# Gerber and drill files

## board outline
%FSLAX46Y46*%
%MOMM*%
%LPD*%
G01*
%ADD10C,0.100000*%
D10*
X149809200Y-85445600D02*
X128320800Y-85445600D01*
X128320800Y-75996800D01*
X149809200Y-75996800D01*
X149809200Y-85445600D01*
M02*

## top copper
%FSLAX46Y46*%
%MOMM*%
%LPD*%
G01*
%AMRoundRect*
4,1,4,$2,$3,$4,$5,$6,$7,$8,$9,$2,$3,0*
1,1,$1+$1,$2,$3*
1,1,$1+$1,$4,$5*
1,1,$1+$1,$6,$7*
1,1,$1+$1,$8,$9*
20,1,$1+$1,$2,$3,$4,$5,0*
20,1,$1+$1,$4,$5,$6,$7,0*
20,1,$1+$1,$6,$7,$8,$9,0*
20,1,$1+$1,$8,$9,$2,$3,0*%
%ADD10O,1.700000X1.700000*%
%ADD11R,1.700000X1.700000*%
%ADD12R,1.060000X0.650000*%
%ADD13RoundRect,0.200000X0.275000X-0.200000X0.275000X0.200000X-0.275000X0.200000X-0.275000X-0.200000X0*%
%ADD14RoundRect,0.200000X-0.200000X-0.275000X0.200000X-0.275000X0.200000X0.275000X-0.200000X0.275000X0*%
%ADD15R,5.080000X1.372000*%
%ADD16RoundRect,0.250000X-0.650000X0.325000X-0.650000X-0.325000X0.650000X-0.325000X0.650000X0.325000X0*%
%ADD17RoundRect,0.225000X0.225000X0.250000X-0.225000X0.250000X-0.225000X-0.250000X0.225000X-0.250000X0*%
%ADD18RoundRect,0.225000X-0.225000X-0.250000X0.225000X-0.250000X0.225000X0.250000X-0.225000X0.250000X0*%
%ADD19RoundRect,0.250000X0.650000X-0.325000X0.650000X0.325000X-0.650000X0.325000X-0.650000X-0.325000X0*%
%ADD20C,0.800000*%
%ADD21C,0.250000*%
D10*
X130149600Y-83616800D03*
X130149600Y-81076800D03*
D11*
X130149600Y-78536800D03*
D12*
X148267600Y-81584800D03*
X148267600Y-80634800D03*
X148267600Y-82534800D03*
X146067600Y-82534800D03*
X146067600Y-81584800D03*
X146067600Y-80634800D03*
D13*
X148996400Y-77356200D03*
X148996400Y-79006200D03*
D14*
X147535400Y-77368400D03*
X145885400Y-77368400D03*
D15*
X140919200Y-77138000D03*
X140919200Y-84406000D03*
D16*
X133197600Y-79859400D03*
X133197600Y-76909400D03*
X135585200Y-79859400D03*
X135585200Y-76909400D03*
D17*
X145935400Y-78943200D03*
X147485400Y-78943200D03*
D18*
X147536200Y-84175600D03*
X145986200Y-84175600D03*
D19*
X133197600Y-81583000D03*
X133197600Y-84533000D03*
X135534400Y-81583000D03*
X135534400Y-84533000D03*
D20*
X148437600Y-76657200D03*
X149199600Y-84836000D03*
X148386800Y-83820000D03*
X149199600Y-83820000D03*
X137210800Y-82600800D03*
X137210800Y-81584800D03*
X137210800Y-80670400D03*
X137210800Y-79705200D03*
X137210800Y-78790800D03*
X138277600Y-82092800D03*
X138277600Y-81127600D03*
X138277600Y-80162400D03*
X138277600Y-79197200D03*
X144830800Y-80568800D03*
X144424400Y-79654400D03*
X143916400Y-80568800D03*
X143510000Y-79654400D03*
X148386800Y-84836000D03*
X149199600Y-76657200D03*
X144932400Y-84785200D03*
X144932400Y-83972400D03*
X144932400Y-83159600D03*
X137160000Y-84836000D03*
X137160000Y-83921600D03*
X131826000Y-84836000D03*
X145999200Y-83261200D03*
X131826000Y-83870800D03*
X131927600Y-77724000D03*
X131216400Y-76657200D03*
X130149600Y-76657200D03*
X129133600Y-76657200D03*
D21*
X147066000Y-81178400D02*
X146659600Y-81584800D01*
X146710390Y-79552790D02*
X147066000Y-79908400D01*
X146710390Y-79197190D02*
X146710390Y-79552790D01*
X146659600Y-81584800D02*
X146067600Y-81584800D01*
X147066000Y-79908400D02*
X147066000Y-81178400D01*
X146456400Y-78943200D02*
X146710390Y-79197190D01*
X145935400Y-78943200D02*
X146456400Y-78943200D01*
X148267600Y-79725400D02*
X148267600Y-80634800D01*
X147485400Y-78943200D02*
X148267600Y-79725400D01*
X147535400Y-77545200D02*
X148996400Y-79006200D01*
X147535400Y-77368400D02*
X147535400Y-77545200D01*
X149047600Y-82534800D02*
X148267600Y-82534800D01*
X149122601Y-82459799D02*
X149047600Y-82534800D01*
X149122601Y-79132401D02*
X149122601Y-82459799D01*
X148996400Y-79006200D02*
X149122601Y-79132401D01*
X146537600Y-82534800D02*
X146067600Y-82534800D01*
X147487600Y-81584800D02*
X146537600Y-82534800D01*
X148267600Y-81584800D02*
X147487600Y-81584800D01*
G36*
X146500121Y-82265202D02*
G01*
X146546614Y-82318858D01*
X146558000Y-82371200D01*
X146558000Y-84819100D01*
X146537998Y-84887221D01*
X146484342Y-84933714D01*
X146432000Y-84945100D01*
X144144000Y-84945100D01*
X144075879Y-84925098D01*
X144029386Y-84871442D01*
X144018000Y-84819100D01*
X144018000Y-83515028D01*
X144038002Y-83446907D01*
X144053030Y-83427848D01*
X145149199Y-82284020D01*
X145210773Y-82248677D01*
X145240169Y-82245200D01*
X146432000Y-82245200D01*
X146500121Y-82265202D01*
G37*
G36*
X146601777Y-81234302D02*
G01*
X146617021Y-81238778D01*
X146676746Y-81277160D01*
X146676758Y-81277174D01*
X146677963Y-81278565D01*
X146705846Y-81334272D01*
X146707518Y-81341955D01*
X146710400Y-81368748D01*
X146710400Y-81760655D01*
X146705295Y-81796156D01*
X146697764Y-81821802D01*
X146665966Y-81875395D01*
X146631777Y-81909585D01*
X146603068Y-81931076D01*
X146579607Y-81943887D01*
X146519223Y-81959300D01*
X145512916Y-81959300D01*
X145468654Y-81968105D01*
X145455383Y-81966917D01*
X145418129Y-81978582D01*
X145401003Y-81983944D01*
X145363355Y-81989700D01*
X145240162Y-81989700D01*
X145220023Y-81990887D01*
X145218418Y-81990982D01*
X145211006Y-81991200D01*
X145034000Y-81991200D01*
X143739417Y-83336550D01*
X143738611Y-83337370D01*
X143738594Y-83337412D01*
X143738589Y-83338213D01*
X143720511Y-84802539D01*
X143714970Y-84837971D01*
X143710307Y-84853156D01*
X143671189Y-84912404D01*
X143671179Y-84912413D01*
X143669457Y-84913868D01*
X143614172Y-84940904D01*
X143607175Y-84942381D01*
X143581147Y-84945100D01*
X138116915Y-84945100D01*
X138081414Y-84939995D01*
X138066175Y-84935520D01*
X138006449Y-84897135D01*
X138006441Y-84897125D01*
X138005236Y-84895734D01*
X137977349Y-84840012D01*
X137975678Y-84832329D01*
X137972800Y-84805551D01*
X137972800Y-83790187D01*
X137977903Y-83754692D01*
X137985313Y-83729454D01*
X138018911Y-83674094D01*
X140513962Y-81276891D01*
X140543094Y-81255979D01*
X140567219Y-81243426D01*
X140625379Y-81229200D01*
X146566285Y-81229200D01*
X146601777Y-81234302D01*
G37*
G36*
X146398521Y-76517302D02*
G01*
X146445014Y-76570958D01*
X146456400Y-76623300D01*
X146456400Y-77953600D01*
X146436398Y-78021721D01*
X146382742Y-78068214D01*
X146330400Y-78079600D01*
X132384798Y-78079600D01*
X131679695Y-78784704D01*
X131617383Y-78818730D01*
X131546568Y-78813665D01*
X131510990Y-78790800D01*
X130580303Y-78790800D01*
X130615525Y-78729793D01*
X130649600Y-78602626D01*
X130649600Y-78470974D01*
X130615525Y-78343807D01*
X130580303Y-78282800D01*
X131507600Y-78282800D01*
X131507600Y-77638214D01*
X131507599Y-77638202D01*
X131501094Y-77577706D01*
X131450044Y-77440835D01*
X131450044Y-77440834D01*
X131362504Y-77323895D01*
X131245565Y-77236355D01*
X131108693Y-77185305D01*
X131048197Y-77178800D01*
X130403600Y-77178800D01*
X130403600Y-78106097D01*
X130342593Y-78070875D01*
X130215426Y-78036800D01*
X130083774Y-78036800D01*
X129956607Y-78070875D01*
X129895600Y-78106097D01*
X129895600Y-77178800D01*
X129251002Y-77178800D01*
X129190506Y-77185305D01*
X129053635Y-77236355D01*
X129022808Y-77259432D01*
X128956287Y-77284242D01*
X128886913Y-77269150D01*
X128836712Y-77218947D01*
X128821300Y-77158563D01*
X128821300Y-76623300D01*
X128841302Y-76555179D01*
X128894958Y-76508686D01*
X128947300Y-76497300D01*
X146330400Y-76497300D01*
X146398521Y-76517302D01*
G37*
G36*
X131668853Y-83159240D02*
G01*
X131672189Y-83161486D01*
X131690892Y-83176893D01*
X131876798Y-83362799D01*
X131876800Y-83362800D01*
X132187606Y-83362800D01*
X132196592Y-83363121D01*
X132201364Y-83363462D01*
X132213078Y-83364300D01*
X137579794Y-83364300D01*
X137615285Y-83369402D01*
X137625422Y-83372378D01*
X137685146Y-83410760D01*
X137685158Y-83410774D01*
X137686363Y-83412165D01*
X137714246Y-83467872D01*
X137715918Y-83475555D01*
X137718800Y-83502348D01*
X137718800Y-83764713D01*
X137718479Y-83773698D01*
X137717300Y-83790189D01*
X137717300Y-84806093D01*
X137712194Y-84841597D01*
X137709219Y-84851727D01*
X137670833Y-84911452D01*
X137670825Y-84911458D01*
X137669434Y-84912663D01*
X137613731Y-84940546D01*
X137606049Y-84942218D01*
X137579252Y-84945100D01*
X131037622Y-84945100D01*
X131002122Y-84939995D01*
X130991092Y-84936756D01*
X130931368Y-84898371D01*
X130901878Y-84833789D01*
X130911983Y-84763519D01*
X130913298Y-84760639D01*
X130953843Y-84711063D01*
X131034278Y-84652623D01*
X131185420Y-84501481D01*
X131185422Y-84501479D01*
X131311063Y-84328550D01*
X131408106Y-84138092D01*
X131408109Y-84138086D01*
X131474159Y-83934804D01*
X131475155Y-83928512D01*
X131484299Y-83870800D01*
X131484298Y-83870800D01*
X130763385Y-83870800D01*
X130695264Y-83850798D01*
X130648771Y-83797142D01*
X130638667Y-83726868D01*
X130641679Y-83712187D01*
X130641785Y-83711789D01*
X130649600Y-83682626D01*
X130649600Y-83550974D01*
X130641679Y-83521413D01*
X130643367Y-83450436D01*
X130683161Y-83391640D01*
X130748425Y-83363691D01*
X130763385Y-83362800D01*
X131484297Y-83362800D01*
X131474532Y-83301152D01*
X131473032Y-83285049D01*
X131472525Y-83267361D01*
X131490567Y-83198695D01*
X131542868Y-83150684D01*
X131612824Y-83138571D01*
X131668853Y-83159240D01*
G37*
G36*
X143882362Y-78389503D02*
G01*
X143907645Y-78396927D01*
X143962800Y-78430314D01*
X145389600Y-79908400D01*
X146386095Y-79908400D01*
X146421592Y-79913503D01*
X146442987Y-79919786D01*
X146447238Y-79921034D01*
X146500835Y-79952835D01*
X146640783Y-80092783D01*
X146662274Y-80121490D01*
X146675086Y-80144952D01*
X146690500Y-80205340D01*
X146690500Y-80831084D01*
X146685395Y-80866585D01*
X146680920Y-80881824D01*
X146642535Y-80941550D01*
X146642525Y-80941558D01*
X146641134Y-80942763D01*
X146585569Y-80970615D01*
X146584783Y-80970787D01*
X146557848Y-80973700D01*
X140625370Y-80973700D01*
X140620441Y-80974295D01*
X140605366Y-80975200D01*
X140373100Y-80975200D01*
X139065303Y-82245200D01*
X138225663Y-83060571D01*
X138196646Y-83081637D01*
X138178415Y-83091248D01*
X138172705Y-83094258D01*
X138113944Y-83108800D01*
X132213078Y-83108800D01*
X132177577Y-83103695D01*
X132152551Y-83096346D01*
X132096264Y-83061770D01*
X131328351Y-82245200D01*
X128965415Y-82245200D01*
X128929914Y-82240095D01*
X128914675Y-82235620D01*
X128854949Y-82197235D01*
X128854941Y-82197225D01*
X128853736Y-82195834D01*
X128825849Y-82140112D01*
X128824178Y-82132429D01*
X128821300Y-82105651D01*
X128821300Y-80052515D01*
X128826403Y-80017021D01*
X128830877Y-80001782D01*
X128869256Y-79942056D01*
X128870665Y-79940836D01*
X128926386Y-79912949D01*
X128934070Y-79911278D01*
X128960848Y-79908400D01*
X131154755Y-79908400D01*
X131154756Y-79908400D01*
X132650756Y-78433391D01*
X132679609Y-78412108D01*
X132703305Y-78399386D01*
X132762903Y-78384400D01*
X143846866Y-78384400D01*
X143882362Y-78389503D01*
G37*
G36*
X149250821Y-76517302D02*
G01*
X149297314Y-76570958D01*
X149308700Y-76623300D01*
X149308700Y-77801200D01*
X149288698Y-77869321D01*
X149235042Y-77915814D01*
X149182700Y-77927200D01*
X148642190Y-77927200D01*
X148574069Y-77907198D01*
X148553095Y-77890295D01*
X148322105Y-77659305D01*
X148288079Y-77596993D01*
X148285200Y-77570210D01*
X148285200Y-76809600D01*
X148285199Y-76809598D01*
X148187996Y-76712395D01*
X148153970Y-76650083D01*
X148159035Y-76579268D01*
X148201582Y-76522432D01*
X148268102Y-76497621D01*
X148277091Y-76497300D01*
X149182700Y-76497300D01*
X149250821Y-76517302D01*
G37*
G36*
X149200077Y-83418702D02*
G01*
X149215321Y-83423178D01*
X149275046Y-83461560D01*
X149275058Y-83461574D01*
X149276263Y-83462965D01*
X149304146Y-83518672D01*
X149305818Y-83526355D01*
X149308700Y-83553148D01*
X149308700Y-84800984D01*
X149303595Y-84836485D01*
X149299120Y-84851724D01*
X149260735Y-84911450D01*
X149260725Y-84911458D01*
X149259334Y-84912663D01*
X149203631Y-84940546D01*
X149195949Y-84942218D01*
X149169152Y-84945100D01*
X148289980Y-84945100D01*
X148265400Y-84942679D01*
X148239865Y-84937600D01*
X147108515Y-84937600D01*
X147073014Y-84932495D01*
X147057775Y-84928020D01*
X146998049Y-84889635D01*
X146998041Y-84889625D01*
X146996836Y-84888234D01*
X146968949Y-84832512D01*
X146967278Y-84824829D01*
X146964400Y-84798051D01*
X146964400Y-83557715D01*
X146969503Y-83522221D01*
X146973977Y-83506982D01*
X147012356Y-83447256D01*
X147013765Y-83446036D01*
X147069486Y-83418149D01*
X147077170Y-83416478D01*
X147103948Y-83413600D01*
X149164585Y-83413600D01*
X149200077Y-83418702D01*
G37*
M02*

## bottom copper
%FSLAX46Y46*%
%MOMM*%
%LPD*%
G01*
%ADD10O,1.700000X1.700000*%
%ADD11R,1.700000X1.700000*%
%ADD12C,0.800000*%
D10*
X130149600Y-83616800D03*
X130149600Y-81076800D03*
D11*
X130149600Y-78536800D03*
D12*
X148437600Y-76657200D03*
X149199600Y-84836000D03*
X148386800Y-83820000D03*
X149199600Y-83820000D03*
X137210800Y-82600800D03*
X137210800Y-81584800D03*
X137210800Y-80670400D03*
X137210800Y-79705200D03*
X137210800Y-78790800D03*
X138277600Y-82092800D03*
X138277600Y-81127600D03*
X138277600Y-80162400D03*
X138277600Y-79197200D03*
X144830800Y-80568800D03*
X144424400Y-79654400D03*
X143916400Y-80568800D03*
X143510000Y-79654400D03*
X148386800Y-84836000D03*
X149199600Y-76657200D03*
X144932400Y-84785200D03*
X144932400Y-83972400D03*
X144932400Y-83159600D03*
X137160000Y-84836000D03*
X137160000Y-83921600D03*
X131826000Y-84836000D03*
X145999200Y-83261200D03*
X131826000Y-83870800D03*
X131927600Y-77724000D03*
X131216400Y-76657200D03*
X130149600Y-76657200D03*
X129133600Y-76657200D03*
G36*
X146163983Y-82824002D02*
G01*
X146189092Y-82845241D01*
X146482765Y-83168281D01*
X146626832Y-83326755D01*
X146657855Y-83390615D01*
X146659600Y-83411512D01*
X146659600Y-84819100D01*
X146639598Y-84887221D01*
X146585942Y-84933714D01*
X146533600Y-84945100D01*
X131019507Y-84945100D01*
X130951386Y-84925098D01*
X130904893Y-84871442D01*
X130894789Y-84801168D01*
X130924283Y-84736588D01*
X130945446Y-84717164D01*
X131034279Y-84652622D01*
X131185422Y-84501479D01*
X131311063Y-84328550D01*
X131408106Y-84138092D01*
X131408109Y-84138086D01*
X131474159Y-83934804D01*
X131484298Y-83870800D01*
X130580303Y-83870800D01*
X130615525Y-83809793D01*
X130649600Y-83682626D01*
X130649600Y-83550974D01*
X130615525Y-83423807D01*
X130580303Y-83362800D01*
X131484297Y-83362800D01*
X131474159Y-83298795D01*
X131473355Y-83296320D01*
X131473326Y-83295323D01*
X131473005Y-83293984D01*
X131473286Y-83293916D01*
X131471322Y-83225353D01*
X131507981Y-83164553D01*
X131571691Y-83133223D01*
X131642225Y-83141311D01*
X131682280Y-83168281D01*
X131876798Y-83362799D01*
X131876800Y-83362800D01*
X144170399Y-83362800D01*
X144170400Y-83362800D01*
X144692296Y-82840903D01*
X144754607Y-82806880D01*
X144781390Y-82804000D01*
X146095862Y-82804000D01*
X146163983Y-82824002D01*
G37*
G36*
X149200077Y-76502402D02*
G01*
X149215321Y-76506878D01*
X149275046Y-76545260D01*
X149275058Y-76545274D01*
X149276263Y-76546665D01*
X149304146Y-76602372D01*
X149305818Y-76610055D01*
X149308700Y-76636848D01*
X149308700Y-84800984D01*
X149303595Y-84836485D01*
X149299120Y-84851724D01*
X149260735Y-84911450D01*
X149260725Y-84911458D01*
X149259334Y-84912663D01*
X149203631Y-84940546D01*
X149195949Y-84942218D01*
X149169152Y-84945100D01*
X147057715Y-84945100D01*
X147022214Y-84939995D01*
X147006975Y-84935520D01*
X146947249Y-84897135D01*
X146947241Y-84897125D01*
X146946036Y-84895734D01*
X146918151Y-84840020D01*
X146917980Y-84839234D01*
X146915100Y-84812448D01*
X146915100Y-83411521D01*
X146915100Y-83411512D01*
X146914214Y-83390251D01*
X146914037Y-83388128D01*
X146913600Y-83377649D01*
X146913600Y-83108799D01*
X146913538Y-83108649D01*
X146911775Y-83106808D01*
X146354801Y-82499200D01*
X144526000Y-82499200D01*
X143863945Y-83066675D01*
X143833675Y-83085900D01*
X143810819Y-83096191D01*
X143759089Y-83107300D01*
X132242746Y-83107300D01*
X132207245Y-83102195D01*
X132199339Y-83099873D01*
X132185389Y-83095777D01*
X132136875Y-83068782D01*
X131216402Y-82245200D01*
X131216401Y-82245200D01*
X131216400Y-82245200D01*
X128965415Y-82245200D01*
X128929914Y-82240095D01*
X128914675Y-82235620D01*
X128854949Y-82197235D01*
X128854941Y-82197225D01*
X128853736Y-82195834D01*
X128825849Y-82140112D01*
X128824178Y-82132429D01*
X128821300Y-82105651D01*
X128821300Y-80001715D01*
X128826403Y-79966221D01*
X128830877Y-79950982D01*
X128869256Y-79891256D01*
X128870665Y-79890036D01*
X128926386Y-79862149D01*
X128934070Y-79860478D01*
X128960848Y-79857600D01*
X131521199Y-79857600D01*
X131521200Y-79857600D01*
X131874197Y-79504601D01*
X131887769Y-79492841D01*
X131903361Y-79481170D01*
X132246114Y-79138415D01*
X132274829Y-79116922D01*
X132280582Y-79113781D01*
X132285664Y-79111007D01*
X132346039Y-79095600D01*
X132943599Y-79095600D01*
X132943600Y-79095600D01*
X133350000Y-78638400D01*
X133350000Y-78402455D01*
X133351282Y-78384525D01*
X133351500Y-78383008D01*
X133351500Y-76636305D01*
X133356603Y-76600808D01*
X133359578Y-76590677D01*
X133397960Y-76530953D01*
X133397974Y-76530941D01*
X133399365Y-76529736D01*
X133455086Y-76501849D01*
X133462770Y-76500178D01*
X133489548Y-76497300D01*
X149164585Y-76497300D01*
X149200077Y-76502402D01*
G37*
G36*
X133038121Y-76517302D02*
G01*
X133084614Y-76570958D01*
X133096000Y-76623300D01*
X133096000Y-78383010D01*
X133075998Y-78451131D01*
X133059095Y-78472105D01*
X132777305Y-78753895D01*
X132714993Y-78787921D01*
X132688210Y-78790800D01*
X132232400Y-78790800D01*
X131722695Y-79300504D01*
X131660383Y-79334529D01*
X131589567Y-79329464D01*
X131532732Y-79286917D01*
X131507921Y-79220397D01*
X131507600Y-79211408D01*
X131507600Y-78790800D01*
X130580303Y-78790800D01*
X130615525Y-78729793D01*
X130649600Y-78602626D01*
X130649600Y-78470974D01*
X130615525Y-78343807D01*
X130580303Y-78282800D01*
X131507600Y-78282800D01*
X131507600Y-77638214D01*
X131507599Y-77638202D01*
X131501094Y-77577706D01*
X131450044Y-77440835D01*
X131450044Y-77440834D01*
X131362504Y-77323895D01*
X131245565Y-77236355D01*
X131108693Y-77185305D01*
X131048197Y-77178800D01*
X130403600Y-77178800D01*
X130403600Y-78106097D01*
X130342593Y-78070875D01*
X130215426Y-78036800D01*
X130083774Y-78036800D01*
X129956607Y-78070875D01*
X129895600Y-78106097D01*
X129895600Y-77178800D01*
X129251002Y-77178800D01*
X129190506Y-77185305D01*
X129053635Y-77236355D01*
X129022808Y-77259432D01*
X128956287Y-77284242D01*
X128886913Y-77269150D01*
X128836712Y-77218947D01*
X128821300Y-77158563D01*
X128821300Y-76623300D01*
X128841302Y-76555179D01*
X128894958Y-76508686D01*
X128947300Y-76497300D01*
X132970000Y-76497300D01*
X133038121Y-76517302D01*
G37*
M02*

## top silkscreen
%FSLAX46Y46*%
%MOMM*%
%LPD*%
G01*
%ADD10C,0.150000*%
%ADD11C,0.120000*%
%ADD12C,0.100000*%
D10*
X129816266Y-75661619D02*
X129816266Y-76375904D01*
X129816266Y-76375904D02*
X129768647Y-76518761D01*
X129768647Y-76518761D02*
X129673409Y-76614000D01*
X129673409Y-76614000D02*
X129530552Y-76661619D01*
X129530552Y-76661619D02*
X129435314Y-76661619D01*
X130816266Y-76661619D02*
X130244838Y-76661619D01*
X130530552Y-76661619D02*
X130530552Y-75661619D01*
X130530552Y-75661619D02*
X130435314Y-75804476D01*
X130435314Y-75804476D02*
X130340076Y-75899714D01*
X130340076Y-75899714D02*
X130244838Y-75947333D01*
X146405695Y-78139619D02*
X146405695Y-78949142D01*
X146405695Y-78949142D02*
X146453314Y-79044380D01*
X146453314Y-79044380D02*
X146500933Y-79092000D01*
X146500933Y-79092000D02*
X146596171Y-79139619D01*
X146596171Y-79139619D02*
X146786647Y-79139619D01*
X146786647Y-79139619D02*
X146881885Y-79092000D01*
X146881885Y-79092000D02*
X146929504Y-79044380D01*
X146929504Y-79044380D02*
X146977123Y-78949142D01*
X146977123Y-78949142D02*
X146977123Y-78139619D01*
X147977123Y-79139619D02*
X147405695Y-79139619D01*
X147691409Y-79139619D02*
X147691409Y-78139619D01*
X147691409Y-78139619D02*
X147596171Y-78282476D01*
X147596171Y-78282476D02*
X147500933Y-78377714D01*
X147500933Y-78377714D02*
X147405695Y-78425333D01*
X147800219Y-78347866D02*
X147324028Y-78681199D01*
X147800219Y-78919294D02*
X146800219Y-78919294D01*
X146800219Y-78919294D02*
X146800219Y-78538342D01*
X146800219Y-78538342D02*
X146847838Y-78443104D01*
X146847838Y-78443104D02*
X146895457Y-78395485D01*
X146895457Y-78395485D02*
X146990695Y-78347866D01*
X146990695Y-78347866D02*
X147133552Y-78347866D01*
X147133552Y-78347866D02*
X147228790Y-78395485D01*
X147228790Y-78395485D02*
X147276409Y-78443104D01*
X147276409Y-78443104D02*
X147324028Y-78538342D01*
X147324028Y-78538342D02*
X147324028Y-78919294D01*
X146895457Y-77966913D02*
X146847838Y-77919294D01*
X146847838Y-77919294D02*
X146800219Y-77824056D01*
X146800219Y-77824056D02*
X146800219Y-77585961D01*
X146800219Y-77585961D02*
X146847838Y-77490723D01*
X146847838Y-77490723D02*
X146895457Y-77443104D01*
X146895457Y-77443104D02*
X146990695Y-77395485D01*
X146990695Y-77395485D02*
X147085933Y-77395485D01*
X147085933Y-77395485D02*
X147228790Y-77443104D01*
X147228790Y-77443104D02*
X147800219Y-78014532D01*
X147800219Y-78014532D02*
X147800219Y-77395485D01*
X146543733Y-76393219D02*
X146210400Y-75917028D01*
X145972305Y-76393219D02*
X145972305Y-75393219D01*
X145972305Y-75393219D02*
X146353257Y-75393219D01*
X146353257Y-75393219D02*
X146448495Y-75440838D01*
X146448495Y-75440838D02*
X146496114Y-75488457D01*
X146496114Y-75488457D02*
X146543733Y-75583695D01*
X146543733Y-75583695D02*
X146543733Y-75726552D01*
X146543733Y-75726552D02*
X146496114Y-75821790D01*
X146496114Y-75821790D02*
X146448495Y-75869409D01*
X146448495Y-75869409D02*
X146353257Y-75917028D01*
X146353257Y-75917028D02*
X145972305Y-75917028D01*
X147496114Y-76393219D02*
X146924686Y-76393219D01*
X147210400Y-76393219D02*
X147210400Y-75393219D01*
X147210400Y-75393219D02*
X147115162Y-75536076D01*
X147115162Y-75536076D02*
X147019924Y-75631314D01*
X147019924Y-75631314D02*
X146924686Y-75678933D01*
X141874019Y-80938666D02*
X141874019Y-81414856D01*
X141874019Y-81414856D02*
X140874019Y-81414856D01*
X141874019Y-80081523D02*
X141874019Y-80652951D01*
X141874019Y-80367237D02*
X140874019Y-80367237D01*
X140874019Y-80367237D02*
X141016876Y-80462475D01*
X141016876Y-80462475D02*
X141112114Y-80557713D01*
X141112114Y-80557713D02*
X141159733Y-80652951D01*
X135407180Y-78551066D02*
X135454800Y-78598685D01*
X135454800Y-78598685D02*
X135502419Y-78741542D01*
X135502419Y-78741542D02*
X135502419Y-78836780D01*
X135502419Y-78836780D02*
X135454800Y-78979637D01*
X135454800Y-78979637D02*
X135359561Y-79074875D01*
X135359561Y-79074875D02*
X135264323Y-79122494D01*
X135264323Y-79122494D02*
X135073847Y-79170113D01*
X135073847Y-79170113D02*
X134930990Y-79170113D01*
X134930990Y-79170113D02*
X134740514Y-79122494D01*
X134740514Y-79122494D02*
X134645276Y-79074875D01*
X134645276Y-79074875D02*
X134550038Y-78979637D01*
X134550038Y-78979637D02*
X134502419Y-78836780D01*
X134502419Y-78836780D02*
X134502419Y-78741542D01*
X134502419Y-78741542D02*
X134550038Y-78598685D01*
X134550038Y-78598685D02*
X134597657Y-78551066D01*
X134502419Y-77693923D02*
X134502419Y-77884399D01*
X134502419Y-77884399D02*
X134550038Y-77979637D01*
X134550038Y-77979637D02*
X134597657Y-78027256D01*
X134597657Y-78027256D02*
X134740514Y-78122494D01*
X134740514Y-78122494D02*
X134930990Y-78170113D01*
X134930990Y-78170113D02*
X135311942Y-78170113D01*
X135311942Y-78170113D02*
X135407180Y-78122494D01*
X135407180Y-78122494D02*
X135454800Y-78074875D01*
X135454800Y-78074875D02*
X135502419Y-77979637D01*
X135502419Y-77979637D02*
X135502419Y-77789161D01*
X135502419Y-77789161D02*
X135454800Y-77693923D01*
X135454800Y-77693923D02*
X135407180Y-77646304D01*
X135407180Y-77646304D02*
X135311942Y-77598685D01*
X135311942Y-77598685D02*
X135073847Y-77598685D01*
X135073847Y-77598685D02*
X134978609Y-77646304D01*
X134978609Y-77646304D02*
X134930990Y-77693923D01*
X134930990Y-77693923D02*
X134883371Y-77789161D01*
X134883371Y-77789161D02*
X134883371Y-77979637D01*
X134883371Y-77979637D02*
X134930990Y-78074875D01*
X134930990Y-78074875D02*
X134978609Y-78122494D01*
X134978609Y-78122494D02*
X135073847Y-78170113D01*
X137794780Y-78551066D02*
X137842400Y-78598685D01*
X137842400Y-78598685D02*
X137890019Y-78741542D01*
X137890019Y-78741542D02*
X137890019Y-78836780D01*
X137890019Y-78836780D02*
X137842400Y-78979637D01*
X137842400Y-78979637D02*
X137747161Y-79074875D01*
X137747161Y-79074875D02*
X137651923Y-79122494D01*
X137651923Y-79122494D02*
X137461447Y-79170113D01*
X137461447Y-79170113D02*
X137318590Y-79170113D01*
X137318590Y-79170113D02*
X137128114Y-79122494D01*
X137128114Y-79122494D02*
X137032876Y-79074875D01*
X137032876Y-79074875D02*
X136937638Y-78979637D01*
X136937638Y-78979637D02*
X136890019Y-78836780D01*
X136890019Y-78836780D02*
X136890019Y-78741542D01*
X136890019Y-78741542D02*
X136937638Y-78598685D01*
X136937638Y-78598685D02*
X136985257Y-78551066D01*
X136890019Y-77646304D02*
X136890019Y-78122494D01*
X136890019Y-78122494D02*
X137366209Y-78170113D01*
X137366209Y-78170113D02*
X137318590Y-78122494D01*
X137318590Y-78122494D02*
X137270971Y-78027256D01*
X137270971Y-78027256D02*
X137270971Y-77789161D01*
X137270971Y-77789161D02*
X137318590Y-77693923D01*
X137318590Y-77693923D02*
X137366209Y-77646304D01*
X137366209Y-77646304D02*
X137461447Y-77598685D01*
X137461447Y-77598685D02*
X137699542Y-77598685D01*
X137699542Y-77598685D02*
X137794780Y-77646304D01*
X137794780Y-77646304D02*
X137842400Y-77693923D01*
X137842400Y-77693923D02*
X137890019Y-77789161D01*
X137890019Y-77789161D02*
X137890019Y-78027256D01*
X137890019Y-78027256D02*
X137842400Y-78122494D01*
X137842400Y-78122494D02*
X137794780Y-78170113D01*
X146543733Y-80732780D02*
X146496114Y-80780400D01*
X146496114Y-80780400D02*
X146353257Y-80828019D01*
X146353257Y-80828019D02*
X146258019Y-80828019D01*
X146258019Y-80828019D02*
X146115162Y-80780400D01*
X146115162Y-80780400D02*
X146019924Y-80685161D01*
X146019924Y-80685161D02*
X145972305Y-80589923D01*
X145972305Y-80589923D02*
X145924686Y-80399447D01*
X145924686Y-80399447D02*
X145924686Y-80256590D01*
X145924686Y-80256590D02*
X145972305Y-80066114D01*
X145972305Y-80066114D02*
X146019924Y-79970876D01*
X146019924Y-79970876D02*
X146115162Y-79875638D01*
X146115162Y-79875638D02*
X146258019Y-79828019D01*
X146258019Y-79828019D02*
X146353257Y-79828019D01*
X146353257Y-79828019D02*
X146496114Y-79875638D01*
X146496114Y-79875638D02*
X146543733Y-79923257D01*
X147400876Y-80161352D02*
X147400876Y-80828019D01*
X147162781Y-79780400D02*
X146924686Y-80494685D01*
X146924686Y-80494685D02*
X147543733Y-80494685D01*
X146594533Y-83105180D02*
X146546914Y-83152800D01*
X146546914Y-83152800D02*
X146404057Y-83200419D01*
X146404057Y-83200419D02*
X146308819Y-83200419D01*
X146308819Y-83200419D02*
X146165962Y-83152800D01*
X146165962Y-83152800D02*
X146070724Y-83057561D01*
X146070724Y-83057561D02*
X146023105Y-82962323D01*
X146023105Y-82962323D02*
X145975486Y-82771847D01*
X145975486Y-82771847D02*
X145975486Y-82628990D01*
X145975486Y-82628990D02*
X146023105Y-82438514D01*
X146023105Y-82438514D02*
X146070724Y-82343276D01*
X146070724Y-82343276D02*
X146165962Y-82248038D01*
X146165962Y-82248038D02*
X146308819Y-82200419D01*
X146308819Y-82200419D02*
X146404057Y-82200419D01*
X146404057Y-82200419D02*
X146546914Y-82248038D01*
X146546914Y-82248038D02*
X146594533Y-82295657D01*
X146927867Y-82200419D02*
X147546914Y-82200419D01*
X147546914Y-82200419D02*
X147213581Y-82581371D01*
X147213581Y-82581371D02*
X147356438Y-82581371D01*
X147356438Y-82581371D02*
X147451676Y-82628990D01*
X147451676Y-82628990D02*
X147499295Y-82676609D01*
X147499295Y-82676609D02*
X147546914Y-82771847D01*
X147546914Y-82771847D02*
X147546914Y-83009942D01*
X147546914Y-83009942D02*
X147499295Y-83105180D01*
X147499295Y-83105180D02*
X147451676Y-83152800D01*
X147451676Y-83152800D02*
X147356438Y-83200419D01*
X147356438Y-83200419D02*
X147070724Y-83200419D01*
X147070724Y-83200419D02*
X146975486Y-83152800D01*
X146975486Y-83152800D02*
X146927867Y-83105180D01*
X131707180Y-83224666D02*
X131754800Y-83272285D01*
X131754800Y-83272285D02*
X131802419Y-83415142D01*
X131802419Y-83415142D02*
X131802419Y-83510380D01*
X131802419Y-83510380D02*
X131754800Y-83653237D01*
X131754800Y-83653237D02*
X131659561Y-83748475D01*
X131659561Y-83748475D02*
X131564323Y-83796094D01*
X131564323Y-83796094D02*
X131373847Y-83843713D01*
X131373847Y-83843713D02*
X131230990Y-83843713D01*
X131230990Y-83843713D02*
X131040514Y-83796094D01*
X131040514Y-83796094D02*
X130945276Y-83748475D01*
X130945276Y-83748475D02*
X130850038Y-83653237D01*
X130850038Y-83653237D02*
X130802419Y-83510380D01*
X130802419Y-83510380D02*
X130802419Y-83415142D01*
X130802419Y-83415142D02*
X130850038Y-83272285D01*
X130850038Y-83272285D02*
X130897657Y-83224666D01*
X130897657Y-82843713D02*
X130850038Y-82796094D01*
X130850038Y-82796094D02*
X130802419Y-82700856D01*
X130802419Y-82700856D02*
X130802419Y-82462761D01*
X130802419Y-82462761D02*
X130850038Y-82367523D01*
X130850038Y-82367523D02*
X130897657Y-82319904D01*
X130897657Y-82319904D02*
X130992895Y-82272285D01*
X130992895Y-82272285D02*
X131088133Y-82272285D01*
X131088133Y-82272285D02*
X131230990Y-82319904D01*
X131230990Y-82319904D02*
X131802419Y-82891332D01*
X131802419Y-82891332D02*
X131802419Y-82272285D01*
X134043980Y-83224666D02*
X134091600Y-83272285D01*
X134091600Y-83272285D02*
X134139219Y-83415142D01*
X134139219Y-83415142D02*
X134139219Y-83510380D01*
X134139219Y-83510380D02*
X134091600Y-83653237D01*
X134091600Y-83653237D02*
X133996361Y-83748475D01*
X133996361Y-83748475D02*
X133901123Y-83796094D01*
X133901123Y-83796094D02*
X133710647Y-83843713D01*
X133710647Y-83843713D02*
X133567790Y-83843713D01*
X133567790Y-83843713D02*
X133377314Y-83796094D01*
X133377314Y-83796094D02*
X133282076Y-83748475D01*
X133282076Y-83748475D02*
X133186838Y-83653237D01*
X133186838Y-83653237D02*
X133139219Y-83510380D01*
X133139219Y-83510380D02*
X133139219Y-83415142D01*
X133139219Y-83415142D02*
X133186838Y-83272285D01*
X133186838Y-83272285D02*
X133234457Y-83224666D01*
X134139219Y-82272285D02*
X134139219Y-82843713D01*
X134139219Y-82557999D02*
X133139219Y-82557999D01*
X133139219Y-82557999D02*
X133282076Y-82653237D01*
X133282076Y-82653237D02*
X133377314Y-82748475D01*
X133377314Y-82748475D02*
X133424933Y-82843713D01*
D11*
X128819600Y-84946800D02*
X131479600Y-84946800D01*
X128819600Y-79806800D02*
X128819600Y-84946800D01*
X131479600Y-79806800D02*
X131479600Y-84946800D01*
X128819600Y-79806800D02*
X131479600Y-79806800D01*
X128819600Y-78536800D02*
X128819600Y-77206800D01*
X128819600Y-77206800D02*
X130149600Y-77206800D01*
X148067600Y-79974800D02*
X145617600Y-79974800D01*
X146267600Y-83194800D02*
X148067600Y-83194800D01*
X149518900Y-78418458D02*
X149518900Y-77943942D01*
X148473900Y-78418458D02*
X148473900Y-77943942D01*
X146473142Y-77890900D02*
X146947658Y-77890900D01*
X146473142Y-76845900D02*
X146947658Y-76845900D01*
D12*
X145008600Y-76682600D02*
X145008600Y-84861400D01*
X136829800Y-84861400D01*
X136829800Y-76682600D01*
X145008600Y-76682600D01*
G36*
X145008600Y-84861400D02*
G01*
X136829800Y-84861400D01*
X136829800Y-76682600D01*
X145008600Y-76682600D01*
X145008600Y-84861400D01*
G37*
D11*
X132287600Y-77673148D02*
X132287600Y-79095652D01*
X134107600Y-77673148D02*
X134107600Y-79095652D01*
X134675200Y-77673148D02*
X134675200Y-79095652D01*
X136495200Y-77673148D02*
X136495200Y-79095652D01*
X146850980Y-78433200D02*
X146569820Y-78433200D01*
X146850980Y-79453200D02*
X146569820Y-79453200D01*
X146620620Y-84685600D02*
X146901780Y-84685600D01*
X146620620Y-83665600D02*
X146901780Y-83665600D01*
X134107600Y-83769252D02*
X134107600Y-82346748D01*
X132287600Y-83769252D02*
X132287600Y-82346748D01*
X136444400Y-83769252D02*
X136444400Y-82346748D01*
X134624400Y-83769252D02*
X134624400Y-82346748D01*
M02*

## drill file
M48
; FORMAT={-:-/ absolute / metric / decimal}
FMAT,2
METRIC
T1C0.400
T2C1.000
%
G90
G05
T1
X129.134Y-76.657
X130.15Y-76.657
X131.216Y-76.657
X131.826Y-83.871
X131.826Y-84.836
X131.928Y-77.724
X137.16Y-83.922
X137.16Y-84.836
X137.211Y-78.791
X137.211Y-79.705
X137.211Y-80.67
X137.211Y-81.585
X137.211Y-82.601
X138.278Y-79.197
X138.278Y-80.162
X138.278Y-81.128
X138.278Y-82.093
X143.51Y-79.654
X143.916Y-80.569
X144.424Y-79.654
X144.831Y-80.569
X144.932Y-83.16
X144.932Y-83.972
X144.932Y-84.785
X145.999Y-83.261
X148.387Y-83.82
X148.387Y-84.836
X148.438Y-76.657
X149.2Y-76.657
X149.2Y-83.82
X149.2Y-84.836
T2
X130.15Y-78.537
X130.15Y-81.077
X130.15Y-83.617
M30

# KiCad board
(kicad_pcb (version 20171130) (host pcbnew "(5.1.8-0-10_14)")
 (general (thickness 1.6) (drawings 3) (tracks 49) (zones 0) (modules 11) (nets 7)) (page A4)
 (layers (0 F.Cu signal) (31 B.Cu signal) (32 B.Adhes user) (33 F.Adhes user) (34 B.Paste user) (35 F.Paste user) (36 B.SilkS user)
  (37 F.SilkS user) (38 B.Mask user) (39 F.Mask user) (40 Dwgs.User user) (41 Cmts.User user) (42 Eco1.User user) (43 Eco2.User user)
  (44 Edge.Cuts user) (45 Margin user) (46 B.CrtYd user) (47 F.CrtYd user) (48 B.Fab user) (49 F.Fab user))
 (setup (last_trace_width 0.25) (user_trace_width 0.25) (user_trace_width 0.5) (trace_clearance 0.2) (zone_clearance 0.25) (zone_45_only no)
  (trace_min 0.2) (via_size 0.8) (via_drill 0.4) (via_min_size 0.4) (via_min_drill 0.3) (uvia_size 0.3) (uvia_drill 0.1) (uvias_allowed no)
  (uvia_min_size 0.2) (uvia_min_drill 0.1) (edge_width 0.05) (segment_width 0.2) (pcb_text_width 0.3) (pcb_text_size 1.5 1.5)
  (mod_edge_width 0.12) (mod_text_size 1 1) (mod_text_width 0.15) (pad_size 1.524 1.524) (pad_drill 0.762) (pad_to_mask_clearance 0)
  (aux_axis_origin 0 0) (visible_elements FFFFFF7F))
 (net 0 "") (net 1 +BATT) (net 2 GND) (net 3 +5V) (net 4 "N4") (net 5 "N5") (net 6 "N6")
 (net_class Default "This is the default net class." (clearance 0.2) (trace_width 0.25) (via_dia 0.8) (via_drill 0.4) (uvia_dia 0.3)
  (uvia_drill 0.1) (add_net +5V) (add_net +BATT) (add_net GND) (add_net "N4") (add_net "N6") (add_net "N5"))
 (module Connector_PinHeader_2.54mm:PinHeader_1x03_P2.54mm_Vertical (layer F.Cu) (at 130.1496 78.5368)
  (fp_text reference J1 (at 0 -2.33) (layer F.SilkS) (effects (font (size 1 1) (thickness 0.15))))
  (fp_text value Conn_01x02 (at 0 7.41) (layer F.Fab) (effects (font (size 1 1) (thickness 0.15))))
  (fp_line (start -1.33 6.41) (end 1.33 6.41) (layer F.SilkS) (width 0.12))
  (fp_line (start -1.33 1.27) (end -1.33 6.41) (layer F.SilkS) (width 0.12))
  (fp_line (start 1.33 1.27) (end 1.33 6.41) (layer F.SilkS) (width 0.12))
  (fp_line (start -1.33 1.27) (end 1.33 1.27) (layer F.SilkS) (width 0.12))
  (fp_line (start -1.33 0) (end -1.33 -1.33) (layer F.SilkS) (width 0.12))
  (fp_line (start -1.33 -1.33) (end 0 -1.33) (layer F.SilkS) (width 0.12))
  (pad 3 thru_hole oval (at 0 5.08) (size 1.7 1.7) (drill 1) (layers *.Cu *.Mask) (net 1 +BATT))
  (pad 2 thru_hole oval (at 0 2.54) (size 1.7 1.7) (drill 1) (layers *.Cu *.Mask) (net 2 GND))
  (pad 1 thru_hole rect (at 0 0) (size 1.7 1.7) (drill 1) (layers *.Cu *.Mask) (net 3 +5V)))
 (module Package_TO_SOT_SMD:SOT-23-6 (layer F.Cu) (at 147.1676 81.5848)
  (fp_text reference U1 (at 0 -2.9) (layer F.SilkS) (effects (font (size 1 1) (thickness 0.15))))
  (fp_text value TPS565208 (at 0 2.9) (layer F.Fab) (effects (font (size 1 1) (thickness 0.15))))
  (fp_line (start 0.9 -1.61) (end -1.55 -1.61) (layer F.SilkS) (width 0.12))
  (fp_line (start -0.9 1.61) (end 0.9 1.61) (layer F.SilkS) (width 0.12))
  (pad 5 smd rect (at 1.1 0) (size 1.06 0.65) (layers F.Cu F.Paste F.Mask) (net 1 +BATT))
  (pad 6 smd rect (at 1.1 -0.95) (size 1.06 0.65) (layers F.Cu F.Paste F.Mask) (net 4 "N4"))
  (pad 4 smd rect (at 1.1 0.95) (size 1.06 0.65) (layers F.Cu F.Paste F.Mask) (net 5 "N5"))
  (pad 3 smd rect (at -1.1 0.95) (size 1.06 0.65) (layers F.Cu F.Paste F.Mask) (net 1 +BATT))
  (pad 2 smd rect (at -1.1 0) (size 1.06 0.65) (layers F.Cu F.Paste F.Mask) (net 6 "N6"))
  (pad 1 smd rect (at -1.1 -0.95) (size 1.06 0.65) (layers F.Cu F.Paste F.Mask) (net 2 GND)))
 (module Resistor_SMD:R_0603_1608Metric (layer F.Cu) (at 148.9964 78.1812 90)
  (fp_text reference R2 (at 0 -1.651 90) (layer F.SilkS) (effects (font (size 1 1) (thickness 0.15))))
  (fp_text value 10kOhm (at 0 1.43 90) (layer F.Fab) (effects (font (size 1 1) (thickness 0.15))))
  (fp_line (start -0.237258 0.5225) (end 0.237258 0.5225) (layer F.SilkS) (width 0.12))
  (fp_line (start -0.237258 -0.5225) (end 0.237258 -0.5225) (layer F.SilkS) (width 0.12))
  (pad 2 smd roundrect (at 0.825 0 90) (size 0.8 0.95) (layers F.Cu F.Paste F.Mask) (roundrect_rratio 0.25) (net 2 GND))
  (pad 1 smd roundrect (at -0.825 0 90) (size 0.8 0.95) (layers F.Cu F.Paste F.Mask) (roundrect_rratio 0.25) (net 5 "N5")))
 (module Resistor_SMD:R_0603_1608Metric (layer F.Cu) (at 146.7104 77.3684)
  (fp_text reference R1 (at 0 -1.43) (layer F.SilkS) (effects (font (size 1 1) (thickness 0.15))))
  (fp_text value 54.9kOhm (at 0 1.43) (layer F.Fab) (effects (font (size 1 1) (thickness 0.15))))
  (fp_line (start -0.237258 0.5225) (end 0.237258 0.5225) (layer F.SilkS) (width 0.12))
  (fp_line (start -0.237258 -0.5225) (end 0.237258 -0.5225) (layer F.SilkS) (width 0.12))
  (pad 2 smd roundrect (at 0.825 0) (size 0.8 0.95) (layers F.Cu F.Paste F.Mask) (roundrect_rratio 0.25) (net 5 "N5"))
  (pad 1 smd roundrect (at -0.825 0) (size 0.8 0.95) (layers F.Cu F.Paste F.Mask) (roundrect_rratio 0.25) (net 3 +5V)))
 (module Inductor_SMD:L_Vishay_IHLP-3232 (layer F.Cu) (at 140.9192 80.772 90)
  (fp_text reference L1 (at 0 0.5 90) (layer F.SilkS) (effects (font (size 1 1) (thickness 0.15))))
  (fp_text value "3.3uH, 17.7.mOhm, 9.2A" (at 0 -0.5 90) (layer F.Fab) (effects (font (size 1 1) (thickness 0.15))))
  (fp_poly (pts (xy 4.0894 4.0894) (xy -4.0894 4.0894) (xy -4.0894 -4.0894) (xy 4.0894 -4.0894)) (layer F.SilkS) (width 0.1))
  (pad 2 smd rect (at 3.634 0 90) (size 1.372 5.08) (layers F.Cu F.Paste F.Mask) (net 3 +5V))
  (pad 1 smd rect (at -3.634 0 90) (size 1.372 5.08) (layers F.Cu F.Paste F.Mask) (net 6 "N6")))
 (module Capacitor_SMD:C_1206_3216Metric (layer F.Cu) (at 133.1976 78.3844 270)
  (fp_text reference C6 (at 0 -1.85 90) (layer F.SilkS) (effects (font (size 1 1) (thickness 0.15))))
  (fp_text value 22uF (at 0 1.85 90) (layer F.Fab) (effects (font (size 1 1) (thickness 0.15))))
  (fp_line (start -0.711252 0.91) (end 0.711252 0.91) (layer F.SilkS) (width 0.12))
  (fp_line (start -0.711252 -0.91) (end 0.711252 -0.91) (layer F.SilkS) (width 0.12))
  (pad 2 smd roundrect (at 1.475 0 270) (size 1.15 1.8) (layers F.Cu F.Paste F.Mask) (roundrect_rratio 0.217391) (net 2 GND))
  (pad 1 smd roundrect (at -1.475 0 270) (size 1.15 1.8) (layers F.Cu F.Paste F.Mask) (roundrect_rratio 0.217391) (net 3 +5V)))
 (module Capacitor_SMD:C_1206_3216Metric (layer F.Cu) (at 135.5852 78.3844 270)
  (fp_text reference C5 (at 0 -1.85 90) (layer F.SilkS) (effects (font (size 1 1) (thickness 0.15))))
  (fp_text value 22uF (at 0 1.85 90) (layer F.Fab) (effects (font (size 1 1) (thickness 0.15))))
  (fp_line (start -0.711252 0.91) (end 0.711252 0.91) (layer F.SilkS) (width 0.12))
  (fp_line (start -0.711252 -0.91) (end 0.711252 -0.91) (layer F.SilkS) (width 0.12))
  (pad 2 smd roundrect (at 1.475 0 270) (size 1.15 1.8) (layers F.Cu F.Paste F.Mask) (roundrect_rratio 0.217391) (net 2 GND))
  (pad 1 smd roundrect (at -1.475 0 270) (size 1.15 1.8) (layers F.Cu F.Paste F.Mask) (roundrect_rratio 0.217391) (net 3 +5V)))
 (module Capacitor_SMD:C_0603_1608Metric (layer F.Cu) (at 146.7104 78.9432 180)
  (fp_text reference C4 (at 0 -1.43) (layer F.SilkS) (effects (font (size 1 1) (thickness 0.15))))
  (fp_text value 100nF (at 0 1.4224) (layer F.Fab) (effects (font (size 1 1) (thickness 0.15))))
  (fp_line (start -0.14058 0.51) (end 0.14058 0.51) (layer F.SilkS) (width 0.12))
  (fp_line (start -0.14058 -0.51) (end 0.14058 -0.51) (layer F.SilkS) (width 0.12))
  (pad 2 smd roundrect (at 0.775 0 180) (size 0.9 0.95) (layers F.Cu F.Paste F.Mask) (roundrect_rratio 0.25) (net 6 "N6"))
  (pad 1 smd roundrect (at -0.775 0 180) (size 0.9 0.95) (layers F.Cu F.Paste F.Mask) (roundrect_rratio 0.25) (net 4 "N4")))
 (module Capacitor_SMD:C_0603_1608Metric (layer F.Cu) (at 146.7612 84.1756)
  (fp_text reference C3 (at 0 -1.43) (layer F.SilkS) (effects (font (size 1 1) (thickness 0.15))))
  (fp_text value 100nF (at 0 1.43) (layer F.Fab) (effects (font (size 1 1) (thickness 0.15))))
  (fp_line (start -0.14058 0.51) (end 0.14058 0.51) (layer F.SilkS) (width 0.12))
  (fp_line (start -0.14058 -0.51) (end 0.14058 -0.51) (layer F.SilkS) (width 0.12))
  (pad 2 smd roundrect (at 0.775 0) (size 0.9 0.95) (layers F.Cu F.Paste F.Mask) (roundrect_rratio 0.25) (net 2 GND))
  (pad 1 smd roundrect (at -0.775 0) (size 0.9 0.95) (layers F.Cu F.Paste F.Mask) (roundrect_rratio 0.25) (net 1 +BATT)))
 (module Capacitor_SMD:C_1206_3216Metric (layer F.Cu) (at 133.1976 83.058 90)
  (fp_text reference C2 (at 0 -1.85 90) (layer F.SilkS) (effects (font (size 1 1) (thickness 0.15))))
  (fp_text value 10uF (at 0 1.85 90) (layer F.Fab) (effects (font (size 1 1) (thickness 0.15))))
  (fp_line (start -0.711252 0.91) (end 0.711252 0.91) (layer F.SilkS) (width 0.12))
  (fp_line (start -0.711252 -0.91) (end 0.711252 -0.91) (layer F.SilkS) (width 0.12))
  (pad 2 smd roundrect (at 1.475 0 90) (size 1.15 1.8) (layers F.Cu F.Paste F.Mask) (roundrect_rratio 0.217391) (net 2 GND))
  (pad 1 smd roundrect (at -1.475 0 90) (size 1.15 1.8) (layers F.Cu F.Paste F.Mask) (roundrect_rratio 0.217391) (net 1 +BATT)))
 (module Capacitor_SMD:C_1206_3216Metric (layer F.Cu) (at 135.5344 83.058 90)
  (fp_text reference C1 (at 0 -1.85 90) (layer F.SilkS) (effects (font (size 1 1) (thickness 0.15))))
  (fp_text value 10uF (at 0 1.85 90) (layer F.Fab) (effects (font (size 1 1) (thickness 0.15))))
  (fp_line (start -0.711252 0.91) (end 0.711252 0.91) (layer F.SilkS) (width 0.12))
  (fp_line (start -0.711252 -0.91) (end 0.711252 -0.91) (layer F.SilkS) (width 0.12))
  (pad 2 smd roundrect (at 1.475 0 90) (size 1.15 1.8) (layers F.Cu F.Paste F.Mask) (roundrect_rratio 0.217391) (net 2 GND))
  (pad 1 smd roundrect (at -1.475 0 90) (size 1.15 1.8) (layers F.Cu F.Paste F.Mask) (roundrect_rratio 0.217391) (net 1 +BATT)))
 (gr_poly (pts (xy 149.8092 85.4456) (xy 128.3208 85.4456) (xy 128.3208 75.9968) (xy 149.8092 75.9968)) (layer Edge.Cuts) (width 0.1))
 (segment (start 147.066 81.1784) (end 146.6596 81.5848) (width 0.25) (layer F.Cu) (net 6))
 (segment (start 146.71039 79.55279) (end 147.066 79.9084) (width 0.25) (layer F.Cu) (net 6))
 (segment (start 146.71039 79.19719) (end 146.71039 79.55279) (width 0.25) (layer F.Cu) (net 6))
 (segment (start 146.6596 81.5848) (end 146.0676 81.5848) (width 0.25) (layer F.Cu) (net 6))
 (segment (start 147.066 79.9084) (end 147.066 81.1784) (width 0.25) (layer F.Cu) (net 6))
 (segment (start 146.4564 78.9432) (end 146.71039 79.19719) (width 0.25) (layer F.Cu) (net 6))
 (segment (start 145.9354 78.9432) (end 146.4564 78.9432) (width 0.25) (layer F.Cu) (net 6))
 (segment (start 148.2676 79.7254) (end 148.2676 80.6348) (width 0.25) (layer F.Cu) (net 4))
 (segment (start 147.4854 78.9432) (end 148.2676 79.7254) (width 0.25) (layer F.Cu) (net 4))
 (segment (start 147.5354 77.5452) (end 148.9964 79.0062) (width 0.25) (layer F.Cu) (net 5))
 (segment (start 147.5354 77.3684) (end 147.5354 77.5452) (width 0.25) (layer F.Cu) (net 5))
 (segment (start 149.0476 82.5348) (end 148.2676 82.5348) (width 0.25) (layer F.Cu) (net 5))
 (segment (start 149.122601 82.459799) (end 149.0476 82.5348) (width 0.25) (layer F.Cu) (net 5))
 (segment (start 149.122601 79.132401) (end 149.122601 82.459799) (width 0.25) (layer F.Cu) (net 5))
 (segment (start 148.9964 79.0062) (end 149.122601 79.132401) (width 0.25) (layer F.Cu) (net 5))
 (via (at 148.4376 76.6572) (size 0.8) (drill 0.4) (layers F.Cu B.Cu) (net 2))
 (via (at 149.1996 84.836) (size 0.8) (drill 0.4) (layers F.Cu B.Cu) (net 2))
 (via (at 148.3868 83.82) (size 0.8) (drill 0.4) (layers F.Cu B.Cu) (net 2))
 (via (at 149.1996 83.82) (size 0.8) (drill 0.4) (layers F.Cu B.Cu) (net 2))
 (via (at 137.2108 82.6008) (size 0.8) (drill 0.4) (layers F.Cu B.Cu) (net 2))
 (via (at 137.2108 81.5848) (size 0.8) (drill 0.4) (layers F.Cu B.Cu) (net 2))
 (via (at 137.2108 80.6704) (size 0.8) (drill 0.4) (layers F.Cu B.Cu) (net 2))
 (via (at 137.2108 79.7052) (size 0.8) (drill 0.4) (layers F.Cu B.Cu) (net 2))
 (via (at 137.2108 78.7908) (size 0.8) (drill 0.4) (layers F.Cu B.Cu) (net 2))
 (via (at 138.2776 82.0928) (size 0.8) (drill 0.4) (layers F.Cu B.Cu) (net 2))
 (via (at 138.2776 81.1276) (size 0.8) (drill 0.4) (layers F.Cu B.Cu) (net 2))
 (via (at 138.2776 80.1624) (size 0.8) (drill 0.4) (layers F.Cu B.Cu) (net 2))
 (via (at 138.2776 79.1972) (size 0.8) (drill 0.4) (layers F.Cu B.Cu) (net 2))
 (via (at 144.8308 80.5688) (size 0.8) (drill 0.4) (layers F.Cu B.Cu) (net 2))
 (via (at 144.4244 79.6544) (size 0.8) (drill 0.4) (layers F.Cu B.Cu) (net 2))
 (via (at 143.9164 80.5688) (size 0.8) (drill 0.4) (layers F.Cu B.Cu) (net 2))
 (via (at 143.51 79.6544) (size 0.8) (drill 0.4) (layers F.Cu B.Cu) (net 2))
 (via (at 148.3868 84.836) (size 0.8) (drill 0.4) (layers F.Cu B.Cu) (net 2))
 (via (at 149.1996 76.6572) (size 0.8) (drill 0.4) (layers F.Cu B.Cu) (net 2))
 (segment (start 146.5376 82.5348) (end 146.0676 82.5348) (width 0.25) (layer F.Cu) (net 1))
 (segment (start 147.4876 81.5848) (end 146.5376 82.5348) (width 0.25) (layer F.Cu) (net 1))
 (segment (start 148.2676 81.5848) (end 147.4876 81.5848) (width 0.25) (layer F.Cu) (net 1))
 (via (at 144.9324 84.7852) (size 0.8) (drill 0.4) (layers F.Cu B.Cu) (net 1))
 (via (at 144.9324 83.9724) (size 0.8) (drill 0.4) (layers F.Cu B.Cu) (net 1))
 (via (at 144.9324 83.1596) (size 0.8) (drill 0.4) (layers F.Cu B.Cu) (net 1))
 (via (at 137.16 84.836) (size 0.8) (drill 0.4) (layers F.Cu B.Cu) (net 1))
 (via (at 137.16 83.9216) (size 0.8) (drill 0.4) (layers F.Cu B.Cu) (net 1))
 (via (at 131.826 84.836) (size 0.8) (drill 0.4) (layers F.Cu B.Cu) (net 1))
 (via (at 145.9992 83.2612) (size 0.8) (drill 0.4) (layers F.Cu B.Cu) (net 1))
 (via (at 131.826 83.8708) (size 0.8) (drill 0.4) (layers F.Cu B.Cu) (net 1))
 (via (at 131.9276 77.724) (size 0.8) (drill 0.4) (layers F.Cu B.Cu) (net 3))
 (via (at 131.2164 76.6572) (size 0.8) (drill 0.4) (layers F.Cu B.Cu) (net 3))
 (via (at 130.1496 76.6572) (size 0.8) (drill 0.4) (layers F.Cu B.Cu) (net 3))
 (via (at 129.1336 76.6572) (size 0.8) (drill 0.4) (layers F.Cu B.Cu) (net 3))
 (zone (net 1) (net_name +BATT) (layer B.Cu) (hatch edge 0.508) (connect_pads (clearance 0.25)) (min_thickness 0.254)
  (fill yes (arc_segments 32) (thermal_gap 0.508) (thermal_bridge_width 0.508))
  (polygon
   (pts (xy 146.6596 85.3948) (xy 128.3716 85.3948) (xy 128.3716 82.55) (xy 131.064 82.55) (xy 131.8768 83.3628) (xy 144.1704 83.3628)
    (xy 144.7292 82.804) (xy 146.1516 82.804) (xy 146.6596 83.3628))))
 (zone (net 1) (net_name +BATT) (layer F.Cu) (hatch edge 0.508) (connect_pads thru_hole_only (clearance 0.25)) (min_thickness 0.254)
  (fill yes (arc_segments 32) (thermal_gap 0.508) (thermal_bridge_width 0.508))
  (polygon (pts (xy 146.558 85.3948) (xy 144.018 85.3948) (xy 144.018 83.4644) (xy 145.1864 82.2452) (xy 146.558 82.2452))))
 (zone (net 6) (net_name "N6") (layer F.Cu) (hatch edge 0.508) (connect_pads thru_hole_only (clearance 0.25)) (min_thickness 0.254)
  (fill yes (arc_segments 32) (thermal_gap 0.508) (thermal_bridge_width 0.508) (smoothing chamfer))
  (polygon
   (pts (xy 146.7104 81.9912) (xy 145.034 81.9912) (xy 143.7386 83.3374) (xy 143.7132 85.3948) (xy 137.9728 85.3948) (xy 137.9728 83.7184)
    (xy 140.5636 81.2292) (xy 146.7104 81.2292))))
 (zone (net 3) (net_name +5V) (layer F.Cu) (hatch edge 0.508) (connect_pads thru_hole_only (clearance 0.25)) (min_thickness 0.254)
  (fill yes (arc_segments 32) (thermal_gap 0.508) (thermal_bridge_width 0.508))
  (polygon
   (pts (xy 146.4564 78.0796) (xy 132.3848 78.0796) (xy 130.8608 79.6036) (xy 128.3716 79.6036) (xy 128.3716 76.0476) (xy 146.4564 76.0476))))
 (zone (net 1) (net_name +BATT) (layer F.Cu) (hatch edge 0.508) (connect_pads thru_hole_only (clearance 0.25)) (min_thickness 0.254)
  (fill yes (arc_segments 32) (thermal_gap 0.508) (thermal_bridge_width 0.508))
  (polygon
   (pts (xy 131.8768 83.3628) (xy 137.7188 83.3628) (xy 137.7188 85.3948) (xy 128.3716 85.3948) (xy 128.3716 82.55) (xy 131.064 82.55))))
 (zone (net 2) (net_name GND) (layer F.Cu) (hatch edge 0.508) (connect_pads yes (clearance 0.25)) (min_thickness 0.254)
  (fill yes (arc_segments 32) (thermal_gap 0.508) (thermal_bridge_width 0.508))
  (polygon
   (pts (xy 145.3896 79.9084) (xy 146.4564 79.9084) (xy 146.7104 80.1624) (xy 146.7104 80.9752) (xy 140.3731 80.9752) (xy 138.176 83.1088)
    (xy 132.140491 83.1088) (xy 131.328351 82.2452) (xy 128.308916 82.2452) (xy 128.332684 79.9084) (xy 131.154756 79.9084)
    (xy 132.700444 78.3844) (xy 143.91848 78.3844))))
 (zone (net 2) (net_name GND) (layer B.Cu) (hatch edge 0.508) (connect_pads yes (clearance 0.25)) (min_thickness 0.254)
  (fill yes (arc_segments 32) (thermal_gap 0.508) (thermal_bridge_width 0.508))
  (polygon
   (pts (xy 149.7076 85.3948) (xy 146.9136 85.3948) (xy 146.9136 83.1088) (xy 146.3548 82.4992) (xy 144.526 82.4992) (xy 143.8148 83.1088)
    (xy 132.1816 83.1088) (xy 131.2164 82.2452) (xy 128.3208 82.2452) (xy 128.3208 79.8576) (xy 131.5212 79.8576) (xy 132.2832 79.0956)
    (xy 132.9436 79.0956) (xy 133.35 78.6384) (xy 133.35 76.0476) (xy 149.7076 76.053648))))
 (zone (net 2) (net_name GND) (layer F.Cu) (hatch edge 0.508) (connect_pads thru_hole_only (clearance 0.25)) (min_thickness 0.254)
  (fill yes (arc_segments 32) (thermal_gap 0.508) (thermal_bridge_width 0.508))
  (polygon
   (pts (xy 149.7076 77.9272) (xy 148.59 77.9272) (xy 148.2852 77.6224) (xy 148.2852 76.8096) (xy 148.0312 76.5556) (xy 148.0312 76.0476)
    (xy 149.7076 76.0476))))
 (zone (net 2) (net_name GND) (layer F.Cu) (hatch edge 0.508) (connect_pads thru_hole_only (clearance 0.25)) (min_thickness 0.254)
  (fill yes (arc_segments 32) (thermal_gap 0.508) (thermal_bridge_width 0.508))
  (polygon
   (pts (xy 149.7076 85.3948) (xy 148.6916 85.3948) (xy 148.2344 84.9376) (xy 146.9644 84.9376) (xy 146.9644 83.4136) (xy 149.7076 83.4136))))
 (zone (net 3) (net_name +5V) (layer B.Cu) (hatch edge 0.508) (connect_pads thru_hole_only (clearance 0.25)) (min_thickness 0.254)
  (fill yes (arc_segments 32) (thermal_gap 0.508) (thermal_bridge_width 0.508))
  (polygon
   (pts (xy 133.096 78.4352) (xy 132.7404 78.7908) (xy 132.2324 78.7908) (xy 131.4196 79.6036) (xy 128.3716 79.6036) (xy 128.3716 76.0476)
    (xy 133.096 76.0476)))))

